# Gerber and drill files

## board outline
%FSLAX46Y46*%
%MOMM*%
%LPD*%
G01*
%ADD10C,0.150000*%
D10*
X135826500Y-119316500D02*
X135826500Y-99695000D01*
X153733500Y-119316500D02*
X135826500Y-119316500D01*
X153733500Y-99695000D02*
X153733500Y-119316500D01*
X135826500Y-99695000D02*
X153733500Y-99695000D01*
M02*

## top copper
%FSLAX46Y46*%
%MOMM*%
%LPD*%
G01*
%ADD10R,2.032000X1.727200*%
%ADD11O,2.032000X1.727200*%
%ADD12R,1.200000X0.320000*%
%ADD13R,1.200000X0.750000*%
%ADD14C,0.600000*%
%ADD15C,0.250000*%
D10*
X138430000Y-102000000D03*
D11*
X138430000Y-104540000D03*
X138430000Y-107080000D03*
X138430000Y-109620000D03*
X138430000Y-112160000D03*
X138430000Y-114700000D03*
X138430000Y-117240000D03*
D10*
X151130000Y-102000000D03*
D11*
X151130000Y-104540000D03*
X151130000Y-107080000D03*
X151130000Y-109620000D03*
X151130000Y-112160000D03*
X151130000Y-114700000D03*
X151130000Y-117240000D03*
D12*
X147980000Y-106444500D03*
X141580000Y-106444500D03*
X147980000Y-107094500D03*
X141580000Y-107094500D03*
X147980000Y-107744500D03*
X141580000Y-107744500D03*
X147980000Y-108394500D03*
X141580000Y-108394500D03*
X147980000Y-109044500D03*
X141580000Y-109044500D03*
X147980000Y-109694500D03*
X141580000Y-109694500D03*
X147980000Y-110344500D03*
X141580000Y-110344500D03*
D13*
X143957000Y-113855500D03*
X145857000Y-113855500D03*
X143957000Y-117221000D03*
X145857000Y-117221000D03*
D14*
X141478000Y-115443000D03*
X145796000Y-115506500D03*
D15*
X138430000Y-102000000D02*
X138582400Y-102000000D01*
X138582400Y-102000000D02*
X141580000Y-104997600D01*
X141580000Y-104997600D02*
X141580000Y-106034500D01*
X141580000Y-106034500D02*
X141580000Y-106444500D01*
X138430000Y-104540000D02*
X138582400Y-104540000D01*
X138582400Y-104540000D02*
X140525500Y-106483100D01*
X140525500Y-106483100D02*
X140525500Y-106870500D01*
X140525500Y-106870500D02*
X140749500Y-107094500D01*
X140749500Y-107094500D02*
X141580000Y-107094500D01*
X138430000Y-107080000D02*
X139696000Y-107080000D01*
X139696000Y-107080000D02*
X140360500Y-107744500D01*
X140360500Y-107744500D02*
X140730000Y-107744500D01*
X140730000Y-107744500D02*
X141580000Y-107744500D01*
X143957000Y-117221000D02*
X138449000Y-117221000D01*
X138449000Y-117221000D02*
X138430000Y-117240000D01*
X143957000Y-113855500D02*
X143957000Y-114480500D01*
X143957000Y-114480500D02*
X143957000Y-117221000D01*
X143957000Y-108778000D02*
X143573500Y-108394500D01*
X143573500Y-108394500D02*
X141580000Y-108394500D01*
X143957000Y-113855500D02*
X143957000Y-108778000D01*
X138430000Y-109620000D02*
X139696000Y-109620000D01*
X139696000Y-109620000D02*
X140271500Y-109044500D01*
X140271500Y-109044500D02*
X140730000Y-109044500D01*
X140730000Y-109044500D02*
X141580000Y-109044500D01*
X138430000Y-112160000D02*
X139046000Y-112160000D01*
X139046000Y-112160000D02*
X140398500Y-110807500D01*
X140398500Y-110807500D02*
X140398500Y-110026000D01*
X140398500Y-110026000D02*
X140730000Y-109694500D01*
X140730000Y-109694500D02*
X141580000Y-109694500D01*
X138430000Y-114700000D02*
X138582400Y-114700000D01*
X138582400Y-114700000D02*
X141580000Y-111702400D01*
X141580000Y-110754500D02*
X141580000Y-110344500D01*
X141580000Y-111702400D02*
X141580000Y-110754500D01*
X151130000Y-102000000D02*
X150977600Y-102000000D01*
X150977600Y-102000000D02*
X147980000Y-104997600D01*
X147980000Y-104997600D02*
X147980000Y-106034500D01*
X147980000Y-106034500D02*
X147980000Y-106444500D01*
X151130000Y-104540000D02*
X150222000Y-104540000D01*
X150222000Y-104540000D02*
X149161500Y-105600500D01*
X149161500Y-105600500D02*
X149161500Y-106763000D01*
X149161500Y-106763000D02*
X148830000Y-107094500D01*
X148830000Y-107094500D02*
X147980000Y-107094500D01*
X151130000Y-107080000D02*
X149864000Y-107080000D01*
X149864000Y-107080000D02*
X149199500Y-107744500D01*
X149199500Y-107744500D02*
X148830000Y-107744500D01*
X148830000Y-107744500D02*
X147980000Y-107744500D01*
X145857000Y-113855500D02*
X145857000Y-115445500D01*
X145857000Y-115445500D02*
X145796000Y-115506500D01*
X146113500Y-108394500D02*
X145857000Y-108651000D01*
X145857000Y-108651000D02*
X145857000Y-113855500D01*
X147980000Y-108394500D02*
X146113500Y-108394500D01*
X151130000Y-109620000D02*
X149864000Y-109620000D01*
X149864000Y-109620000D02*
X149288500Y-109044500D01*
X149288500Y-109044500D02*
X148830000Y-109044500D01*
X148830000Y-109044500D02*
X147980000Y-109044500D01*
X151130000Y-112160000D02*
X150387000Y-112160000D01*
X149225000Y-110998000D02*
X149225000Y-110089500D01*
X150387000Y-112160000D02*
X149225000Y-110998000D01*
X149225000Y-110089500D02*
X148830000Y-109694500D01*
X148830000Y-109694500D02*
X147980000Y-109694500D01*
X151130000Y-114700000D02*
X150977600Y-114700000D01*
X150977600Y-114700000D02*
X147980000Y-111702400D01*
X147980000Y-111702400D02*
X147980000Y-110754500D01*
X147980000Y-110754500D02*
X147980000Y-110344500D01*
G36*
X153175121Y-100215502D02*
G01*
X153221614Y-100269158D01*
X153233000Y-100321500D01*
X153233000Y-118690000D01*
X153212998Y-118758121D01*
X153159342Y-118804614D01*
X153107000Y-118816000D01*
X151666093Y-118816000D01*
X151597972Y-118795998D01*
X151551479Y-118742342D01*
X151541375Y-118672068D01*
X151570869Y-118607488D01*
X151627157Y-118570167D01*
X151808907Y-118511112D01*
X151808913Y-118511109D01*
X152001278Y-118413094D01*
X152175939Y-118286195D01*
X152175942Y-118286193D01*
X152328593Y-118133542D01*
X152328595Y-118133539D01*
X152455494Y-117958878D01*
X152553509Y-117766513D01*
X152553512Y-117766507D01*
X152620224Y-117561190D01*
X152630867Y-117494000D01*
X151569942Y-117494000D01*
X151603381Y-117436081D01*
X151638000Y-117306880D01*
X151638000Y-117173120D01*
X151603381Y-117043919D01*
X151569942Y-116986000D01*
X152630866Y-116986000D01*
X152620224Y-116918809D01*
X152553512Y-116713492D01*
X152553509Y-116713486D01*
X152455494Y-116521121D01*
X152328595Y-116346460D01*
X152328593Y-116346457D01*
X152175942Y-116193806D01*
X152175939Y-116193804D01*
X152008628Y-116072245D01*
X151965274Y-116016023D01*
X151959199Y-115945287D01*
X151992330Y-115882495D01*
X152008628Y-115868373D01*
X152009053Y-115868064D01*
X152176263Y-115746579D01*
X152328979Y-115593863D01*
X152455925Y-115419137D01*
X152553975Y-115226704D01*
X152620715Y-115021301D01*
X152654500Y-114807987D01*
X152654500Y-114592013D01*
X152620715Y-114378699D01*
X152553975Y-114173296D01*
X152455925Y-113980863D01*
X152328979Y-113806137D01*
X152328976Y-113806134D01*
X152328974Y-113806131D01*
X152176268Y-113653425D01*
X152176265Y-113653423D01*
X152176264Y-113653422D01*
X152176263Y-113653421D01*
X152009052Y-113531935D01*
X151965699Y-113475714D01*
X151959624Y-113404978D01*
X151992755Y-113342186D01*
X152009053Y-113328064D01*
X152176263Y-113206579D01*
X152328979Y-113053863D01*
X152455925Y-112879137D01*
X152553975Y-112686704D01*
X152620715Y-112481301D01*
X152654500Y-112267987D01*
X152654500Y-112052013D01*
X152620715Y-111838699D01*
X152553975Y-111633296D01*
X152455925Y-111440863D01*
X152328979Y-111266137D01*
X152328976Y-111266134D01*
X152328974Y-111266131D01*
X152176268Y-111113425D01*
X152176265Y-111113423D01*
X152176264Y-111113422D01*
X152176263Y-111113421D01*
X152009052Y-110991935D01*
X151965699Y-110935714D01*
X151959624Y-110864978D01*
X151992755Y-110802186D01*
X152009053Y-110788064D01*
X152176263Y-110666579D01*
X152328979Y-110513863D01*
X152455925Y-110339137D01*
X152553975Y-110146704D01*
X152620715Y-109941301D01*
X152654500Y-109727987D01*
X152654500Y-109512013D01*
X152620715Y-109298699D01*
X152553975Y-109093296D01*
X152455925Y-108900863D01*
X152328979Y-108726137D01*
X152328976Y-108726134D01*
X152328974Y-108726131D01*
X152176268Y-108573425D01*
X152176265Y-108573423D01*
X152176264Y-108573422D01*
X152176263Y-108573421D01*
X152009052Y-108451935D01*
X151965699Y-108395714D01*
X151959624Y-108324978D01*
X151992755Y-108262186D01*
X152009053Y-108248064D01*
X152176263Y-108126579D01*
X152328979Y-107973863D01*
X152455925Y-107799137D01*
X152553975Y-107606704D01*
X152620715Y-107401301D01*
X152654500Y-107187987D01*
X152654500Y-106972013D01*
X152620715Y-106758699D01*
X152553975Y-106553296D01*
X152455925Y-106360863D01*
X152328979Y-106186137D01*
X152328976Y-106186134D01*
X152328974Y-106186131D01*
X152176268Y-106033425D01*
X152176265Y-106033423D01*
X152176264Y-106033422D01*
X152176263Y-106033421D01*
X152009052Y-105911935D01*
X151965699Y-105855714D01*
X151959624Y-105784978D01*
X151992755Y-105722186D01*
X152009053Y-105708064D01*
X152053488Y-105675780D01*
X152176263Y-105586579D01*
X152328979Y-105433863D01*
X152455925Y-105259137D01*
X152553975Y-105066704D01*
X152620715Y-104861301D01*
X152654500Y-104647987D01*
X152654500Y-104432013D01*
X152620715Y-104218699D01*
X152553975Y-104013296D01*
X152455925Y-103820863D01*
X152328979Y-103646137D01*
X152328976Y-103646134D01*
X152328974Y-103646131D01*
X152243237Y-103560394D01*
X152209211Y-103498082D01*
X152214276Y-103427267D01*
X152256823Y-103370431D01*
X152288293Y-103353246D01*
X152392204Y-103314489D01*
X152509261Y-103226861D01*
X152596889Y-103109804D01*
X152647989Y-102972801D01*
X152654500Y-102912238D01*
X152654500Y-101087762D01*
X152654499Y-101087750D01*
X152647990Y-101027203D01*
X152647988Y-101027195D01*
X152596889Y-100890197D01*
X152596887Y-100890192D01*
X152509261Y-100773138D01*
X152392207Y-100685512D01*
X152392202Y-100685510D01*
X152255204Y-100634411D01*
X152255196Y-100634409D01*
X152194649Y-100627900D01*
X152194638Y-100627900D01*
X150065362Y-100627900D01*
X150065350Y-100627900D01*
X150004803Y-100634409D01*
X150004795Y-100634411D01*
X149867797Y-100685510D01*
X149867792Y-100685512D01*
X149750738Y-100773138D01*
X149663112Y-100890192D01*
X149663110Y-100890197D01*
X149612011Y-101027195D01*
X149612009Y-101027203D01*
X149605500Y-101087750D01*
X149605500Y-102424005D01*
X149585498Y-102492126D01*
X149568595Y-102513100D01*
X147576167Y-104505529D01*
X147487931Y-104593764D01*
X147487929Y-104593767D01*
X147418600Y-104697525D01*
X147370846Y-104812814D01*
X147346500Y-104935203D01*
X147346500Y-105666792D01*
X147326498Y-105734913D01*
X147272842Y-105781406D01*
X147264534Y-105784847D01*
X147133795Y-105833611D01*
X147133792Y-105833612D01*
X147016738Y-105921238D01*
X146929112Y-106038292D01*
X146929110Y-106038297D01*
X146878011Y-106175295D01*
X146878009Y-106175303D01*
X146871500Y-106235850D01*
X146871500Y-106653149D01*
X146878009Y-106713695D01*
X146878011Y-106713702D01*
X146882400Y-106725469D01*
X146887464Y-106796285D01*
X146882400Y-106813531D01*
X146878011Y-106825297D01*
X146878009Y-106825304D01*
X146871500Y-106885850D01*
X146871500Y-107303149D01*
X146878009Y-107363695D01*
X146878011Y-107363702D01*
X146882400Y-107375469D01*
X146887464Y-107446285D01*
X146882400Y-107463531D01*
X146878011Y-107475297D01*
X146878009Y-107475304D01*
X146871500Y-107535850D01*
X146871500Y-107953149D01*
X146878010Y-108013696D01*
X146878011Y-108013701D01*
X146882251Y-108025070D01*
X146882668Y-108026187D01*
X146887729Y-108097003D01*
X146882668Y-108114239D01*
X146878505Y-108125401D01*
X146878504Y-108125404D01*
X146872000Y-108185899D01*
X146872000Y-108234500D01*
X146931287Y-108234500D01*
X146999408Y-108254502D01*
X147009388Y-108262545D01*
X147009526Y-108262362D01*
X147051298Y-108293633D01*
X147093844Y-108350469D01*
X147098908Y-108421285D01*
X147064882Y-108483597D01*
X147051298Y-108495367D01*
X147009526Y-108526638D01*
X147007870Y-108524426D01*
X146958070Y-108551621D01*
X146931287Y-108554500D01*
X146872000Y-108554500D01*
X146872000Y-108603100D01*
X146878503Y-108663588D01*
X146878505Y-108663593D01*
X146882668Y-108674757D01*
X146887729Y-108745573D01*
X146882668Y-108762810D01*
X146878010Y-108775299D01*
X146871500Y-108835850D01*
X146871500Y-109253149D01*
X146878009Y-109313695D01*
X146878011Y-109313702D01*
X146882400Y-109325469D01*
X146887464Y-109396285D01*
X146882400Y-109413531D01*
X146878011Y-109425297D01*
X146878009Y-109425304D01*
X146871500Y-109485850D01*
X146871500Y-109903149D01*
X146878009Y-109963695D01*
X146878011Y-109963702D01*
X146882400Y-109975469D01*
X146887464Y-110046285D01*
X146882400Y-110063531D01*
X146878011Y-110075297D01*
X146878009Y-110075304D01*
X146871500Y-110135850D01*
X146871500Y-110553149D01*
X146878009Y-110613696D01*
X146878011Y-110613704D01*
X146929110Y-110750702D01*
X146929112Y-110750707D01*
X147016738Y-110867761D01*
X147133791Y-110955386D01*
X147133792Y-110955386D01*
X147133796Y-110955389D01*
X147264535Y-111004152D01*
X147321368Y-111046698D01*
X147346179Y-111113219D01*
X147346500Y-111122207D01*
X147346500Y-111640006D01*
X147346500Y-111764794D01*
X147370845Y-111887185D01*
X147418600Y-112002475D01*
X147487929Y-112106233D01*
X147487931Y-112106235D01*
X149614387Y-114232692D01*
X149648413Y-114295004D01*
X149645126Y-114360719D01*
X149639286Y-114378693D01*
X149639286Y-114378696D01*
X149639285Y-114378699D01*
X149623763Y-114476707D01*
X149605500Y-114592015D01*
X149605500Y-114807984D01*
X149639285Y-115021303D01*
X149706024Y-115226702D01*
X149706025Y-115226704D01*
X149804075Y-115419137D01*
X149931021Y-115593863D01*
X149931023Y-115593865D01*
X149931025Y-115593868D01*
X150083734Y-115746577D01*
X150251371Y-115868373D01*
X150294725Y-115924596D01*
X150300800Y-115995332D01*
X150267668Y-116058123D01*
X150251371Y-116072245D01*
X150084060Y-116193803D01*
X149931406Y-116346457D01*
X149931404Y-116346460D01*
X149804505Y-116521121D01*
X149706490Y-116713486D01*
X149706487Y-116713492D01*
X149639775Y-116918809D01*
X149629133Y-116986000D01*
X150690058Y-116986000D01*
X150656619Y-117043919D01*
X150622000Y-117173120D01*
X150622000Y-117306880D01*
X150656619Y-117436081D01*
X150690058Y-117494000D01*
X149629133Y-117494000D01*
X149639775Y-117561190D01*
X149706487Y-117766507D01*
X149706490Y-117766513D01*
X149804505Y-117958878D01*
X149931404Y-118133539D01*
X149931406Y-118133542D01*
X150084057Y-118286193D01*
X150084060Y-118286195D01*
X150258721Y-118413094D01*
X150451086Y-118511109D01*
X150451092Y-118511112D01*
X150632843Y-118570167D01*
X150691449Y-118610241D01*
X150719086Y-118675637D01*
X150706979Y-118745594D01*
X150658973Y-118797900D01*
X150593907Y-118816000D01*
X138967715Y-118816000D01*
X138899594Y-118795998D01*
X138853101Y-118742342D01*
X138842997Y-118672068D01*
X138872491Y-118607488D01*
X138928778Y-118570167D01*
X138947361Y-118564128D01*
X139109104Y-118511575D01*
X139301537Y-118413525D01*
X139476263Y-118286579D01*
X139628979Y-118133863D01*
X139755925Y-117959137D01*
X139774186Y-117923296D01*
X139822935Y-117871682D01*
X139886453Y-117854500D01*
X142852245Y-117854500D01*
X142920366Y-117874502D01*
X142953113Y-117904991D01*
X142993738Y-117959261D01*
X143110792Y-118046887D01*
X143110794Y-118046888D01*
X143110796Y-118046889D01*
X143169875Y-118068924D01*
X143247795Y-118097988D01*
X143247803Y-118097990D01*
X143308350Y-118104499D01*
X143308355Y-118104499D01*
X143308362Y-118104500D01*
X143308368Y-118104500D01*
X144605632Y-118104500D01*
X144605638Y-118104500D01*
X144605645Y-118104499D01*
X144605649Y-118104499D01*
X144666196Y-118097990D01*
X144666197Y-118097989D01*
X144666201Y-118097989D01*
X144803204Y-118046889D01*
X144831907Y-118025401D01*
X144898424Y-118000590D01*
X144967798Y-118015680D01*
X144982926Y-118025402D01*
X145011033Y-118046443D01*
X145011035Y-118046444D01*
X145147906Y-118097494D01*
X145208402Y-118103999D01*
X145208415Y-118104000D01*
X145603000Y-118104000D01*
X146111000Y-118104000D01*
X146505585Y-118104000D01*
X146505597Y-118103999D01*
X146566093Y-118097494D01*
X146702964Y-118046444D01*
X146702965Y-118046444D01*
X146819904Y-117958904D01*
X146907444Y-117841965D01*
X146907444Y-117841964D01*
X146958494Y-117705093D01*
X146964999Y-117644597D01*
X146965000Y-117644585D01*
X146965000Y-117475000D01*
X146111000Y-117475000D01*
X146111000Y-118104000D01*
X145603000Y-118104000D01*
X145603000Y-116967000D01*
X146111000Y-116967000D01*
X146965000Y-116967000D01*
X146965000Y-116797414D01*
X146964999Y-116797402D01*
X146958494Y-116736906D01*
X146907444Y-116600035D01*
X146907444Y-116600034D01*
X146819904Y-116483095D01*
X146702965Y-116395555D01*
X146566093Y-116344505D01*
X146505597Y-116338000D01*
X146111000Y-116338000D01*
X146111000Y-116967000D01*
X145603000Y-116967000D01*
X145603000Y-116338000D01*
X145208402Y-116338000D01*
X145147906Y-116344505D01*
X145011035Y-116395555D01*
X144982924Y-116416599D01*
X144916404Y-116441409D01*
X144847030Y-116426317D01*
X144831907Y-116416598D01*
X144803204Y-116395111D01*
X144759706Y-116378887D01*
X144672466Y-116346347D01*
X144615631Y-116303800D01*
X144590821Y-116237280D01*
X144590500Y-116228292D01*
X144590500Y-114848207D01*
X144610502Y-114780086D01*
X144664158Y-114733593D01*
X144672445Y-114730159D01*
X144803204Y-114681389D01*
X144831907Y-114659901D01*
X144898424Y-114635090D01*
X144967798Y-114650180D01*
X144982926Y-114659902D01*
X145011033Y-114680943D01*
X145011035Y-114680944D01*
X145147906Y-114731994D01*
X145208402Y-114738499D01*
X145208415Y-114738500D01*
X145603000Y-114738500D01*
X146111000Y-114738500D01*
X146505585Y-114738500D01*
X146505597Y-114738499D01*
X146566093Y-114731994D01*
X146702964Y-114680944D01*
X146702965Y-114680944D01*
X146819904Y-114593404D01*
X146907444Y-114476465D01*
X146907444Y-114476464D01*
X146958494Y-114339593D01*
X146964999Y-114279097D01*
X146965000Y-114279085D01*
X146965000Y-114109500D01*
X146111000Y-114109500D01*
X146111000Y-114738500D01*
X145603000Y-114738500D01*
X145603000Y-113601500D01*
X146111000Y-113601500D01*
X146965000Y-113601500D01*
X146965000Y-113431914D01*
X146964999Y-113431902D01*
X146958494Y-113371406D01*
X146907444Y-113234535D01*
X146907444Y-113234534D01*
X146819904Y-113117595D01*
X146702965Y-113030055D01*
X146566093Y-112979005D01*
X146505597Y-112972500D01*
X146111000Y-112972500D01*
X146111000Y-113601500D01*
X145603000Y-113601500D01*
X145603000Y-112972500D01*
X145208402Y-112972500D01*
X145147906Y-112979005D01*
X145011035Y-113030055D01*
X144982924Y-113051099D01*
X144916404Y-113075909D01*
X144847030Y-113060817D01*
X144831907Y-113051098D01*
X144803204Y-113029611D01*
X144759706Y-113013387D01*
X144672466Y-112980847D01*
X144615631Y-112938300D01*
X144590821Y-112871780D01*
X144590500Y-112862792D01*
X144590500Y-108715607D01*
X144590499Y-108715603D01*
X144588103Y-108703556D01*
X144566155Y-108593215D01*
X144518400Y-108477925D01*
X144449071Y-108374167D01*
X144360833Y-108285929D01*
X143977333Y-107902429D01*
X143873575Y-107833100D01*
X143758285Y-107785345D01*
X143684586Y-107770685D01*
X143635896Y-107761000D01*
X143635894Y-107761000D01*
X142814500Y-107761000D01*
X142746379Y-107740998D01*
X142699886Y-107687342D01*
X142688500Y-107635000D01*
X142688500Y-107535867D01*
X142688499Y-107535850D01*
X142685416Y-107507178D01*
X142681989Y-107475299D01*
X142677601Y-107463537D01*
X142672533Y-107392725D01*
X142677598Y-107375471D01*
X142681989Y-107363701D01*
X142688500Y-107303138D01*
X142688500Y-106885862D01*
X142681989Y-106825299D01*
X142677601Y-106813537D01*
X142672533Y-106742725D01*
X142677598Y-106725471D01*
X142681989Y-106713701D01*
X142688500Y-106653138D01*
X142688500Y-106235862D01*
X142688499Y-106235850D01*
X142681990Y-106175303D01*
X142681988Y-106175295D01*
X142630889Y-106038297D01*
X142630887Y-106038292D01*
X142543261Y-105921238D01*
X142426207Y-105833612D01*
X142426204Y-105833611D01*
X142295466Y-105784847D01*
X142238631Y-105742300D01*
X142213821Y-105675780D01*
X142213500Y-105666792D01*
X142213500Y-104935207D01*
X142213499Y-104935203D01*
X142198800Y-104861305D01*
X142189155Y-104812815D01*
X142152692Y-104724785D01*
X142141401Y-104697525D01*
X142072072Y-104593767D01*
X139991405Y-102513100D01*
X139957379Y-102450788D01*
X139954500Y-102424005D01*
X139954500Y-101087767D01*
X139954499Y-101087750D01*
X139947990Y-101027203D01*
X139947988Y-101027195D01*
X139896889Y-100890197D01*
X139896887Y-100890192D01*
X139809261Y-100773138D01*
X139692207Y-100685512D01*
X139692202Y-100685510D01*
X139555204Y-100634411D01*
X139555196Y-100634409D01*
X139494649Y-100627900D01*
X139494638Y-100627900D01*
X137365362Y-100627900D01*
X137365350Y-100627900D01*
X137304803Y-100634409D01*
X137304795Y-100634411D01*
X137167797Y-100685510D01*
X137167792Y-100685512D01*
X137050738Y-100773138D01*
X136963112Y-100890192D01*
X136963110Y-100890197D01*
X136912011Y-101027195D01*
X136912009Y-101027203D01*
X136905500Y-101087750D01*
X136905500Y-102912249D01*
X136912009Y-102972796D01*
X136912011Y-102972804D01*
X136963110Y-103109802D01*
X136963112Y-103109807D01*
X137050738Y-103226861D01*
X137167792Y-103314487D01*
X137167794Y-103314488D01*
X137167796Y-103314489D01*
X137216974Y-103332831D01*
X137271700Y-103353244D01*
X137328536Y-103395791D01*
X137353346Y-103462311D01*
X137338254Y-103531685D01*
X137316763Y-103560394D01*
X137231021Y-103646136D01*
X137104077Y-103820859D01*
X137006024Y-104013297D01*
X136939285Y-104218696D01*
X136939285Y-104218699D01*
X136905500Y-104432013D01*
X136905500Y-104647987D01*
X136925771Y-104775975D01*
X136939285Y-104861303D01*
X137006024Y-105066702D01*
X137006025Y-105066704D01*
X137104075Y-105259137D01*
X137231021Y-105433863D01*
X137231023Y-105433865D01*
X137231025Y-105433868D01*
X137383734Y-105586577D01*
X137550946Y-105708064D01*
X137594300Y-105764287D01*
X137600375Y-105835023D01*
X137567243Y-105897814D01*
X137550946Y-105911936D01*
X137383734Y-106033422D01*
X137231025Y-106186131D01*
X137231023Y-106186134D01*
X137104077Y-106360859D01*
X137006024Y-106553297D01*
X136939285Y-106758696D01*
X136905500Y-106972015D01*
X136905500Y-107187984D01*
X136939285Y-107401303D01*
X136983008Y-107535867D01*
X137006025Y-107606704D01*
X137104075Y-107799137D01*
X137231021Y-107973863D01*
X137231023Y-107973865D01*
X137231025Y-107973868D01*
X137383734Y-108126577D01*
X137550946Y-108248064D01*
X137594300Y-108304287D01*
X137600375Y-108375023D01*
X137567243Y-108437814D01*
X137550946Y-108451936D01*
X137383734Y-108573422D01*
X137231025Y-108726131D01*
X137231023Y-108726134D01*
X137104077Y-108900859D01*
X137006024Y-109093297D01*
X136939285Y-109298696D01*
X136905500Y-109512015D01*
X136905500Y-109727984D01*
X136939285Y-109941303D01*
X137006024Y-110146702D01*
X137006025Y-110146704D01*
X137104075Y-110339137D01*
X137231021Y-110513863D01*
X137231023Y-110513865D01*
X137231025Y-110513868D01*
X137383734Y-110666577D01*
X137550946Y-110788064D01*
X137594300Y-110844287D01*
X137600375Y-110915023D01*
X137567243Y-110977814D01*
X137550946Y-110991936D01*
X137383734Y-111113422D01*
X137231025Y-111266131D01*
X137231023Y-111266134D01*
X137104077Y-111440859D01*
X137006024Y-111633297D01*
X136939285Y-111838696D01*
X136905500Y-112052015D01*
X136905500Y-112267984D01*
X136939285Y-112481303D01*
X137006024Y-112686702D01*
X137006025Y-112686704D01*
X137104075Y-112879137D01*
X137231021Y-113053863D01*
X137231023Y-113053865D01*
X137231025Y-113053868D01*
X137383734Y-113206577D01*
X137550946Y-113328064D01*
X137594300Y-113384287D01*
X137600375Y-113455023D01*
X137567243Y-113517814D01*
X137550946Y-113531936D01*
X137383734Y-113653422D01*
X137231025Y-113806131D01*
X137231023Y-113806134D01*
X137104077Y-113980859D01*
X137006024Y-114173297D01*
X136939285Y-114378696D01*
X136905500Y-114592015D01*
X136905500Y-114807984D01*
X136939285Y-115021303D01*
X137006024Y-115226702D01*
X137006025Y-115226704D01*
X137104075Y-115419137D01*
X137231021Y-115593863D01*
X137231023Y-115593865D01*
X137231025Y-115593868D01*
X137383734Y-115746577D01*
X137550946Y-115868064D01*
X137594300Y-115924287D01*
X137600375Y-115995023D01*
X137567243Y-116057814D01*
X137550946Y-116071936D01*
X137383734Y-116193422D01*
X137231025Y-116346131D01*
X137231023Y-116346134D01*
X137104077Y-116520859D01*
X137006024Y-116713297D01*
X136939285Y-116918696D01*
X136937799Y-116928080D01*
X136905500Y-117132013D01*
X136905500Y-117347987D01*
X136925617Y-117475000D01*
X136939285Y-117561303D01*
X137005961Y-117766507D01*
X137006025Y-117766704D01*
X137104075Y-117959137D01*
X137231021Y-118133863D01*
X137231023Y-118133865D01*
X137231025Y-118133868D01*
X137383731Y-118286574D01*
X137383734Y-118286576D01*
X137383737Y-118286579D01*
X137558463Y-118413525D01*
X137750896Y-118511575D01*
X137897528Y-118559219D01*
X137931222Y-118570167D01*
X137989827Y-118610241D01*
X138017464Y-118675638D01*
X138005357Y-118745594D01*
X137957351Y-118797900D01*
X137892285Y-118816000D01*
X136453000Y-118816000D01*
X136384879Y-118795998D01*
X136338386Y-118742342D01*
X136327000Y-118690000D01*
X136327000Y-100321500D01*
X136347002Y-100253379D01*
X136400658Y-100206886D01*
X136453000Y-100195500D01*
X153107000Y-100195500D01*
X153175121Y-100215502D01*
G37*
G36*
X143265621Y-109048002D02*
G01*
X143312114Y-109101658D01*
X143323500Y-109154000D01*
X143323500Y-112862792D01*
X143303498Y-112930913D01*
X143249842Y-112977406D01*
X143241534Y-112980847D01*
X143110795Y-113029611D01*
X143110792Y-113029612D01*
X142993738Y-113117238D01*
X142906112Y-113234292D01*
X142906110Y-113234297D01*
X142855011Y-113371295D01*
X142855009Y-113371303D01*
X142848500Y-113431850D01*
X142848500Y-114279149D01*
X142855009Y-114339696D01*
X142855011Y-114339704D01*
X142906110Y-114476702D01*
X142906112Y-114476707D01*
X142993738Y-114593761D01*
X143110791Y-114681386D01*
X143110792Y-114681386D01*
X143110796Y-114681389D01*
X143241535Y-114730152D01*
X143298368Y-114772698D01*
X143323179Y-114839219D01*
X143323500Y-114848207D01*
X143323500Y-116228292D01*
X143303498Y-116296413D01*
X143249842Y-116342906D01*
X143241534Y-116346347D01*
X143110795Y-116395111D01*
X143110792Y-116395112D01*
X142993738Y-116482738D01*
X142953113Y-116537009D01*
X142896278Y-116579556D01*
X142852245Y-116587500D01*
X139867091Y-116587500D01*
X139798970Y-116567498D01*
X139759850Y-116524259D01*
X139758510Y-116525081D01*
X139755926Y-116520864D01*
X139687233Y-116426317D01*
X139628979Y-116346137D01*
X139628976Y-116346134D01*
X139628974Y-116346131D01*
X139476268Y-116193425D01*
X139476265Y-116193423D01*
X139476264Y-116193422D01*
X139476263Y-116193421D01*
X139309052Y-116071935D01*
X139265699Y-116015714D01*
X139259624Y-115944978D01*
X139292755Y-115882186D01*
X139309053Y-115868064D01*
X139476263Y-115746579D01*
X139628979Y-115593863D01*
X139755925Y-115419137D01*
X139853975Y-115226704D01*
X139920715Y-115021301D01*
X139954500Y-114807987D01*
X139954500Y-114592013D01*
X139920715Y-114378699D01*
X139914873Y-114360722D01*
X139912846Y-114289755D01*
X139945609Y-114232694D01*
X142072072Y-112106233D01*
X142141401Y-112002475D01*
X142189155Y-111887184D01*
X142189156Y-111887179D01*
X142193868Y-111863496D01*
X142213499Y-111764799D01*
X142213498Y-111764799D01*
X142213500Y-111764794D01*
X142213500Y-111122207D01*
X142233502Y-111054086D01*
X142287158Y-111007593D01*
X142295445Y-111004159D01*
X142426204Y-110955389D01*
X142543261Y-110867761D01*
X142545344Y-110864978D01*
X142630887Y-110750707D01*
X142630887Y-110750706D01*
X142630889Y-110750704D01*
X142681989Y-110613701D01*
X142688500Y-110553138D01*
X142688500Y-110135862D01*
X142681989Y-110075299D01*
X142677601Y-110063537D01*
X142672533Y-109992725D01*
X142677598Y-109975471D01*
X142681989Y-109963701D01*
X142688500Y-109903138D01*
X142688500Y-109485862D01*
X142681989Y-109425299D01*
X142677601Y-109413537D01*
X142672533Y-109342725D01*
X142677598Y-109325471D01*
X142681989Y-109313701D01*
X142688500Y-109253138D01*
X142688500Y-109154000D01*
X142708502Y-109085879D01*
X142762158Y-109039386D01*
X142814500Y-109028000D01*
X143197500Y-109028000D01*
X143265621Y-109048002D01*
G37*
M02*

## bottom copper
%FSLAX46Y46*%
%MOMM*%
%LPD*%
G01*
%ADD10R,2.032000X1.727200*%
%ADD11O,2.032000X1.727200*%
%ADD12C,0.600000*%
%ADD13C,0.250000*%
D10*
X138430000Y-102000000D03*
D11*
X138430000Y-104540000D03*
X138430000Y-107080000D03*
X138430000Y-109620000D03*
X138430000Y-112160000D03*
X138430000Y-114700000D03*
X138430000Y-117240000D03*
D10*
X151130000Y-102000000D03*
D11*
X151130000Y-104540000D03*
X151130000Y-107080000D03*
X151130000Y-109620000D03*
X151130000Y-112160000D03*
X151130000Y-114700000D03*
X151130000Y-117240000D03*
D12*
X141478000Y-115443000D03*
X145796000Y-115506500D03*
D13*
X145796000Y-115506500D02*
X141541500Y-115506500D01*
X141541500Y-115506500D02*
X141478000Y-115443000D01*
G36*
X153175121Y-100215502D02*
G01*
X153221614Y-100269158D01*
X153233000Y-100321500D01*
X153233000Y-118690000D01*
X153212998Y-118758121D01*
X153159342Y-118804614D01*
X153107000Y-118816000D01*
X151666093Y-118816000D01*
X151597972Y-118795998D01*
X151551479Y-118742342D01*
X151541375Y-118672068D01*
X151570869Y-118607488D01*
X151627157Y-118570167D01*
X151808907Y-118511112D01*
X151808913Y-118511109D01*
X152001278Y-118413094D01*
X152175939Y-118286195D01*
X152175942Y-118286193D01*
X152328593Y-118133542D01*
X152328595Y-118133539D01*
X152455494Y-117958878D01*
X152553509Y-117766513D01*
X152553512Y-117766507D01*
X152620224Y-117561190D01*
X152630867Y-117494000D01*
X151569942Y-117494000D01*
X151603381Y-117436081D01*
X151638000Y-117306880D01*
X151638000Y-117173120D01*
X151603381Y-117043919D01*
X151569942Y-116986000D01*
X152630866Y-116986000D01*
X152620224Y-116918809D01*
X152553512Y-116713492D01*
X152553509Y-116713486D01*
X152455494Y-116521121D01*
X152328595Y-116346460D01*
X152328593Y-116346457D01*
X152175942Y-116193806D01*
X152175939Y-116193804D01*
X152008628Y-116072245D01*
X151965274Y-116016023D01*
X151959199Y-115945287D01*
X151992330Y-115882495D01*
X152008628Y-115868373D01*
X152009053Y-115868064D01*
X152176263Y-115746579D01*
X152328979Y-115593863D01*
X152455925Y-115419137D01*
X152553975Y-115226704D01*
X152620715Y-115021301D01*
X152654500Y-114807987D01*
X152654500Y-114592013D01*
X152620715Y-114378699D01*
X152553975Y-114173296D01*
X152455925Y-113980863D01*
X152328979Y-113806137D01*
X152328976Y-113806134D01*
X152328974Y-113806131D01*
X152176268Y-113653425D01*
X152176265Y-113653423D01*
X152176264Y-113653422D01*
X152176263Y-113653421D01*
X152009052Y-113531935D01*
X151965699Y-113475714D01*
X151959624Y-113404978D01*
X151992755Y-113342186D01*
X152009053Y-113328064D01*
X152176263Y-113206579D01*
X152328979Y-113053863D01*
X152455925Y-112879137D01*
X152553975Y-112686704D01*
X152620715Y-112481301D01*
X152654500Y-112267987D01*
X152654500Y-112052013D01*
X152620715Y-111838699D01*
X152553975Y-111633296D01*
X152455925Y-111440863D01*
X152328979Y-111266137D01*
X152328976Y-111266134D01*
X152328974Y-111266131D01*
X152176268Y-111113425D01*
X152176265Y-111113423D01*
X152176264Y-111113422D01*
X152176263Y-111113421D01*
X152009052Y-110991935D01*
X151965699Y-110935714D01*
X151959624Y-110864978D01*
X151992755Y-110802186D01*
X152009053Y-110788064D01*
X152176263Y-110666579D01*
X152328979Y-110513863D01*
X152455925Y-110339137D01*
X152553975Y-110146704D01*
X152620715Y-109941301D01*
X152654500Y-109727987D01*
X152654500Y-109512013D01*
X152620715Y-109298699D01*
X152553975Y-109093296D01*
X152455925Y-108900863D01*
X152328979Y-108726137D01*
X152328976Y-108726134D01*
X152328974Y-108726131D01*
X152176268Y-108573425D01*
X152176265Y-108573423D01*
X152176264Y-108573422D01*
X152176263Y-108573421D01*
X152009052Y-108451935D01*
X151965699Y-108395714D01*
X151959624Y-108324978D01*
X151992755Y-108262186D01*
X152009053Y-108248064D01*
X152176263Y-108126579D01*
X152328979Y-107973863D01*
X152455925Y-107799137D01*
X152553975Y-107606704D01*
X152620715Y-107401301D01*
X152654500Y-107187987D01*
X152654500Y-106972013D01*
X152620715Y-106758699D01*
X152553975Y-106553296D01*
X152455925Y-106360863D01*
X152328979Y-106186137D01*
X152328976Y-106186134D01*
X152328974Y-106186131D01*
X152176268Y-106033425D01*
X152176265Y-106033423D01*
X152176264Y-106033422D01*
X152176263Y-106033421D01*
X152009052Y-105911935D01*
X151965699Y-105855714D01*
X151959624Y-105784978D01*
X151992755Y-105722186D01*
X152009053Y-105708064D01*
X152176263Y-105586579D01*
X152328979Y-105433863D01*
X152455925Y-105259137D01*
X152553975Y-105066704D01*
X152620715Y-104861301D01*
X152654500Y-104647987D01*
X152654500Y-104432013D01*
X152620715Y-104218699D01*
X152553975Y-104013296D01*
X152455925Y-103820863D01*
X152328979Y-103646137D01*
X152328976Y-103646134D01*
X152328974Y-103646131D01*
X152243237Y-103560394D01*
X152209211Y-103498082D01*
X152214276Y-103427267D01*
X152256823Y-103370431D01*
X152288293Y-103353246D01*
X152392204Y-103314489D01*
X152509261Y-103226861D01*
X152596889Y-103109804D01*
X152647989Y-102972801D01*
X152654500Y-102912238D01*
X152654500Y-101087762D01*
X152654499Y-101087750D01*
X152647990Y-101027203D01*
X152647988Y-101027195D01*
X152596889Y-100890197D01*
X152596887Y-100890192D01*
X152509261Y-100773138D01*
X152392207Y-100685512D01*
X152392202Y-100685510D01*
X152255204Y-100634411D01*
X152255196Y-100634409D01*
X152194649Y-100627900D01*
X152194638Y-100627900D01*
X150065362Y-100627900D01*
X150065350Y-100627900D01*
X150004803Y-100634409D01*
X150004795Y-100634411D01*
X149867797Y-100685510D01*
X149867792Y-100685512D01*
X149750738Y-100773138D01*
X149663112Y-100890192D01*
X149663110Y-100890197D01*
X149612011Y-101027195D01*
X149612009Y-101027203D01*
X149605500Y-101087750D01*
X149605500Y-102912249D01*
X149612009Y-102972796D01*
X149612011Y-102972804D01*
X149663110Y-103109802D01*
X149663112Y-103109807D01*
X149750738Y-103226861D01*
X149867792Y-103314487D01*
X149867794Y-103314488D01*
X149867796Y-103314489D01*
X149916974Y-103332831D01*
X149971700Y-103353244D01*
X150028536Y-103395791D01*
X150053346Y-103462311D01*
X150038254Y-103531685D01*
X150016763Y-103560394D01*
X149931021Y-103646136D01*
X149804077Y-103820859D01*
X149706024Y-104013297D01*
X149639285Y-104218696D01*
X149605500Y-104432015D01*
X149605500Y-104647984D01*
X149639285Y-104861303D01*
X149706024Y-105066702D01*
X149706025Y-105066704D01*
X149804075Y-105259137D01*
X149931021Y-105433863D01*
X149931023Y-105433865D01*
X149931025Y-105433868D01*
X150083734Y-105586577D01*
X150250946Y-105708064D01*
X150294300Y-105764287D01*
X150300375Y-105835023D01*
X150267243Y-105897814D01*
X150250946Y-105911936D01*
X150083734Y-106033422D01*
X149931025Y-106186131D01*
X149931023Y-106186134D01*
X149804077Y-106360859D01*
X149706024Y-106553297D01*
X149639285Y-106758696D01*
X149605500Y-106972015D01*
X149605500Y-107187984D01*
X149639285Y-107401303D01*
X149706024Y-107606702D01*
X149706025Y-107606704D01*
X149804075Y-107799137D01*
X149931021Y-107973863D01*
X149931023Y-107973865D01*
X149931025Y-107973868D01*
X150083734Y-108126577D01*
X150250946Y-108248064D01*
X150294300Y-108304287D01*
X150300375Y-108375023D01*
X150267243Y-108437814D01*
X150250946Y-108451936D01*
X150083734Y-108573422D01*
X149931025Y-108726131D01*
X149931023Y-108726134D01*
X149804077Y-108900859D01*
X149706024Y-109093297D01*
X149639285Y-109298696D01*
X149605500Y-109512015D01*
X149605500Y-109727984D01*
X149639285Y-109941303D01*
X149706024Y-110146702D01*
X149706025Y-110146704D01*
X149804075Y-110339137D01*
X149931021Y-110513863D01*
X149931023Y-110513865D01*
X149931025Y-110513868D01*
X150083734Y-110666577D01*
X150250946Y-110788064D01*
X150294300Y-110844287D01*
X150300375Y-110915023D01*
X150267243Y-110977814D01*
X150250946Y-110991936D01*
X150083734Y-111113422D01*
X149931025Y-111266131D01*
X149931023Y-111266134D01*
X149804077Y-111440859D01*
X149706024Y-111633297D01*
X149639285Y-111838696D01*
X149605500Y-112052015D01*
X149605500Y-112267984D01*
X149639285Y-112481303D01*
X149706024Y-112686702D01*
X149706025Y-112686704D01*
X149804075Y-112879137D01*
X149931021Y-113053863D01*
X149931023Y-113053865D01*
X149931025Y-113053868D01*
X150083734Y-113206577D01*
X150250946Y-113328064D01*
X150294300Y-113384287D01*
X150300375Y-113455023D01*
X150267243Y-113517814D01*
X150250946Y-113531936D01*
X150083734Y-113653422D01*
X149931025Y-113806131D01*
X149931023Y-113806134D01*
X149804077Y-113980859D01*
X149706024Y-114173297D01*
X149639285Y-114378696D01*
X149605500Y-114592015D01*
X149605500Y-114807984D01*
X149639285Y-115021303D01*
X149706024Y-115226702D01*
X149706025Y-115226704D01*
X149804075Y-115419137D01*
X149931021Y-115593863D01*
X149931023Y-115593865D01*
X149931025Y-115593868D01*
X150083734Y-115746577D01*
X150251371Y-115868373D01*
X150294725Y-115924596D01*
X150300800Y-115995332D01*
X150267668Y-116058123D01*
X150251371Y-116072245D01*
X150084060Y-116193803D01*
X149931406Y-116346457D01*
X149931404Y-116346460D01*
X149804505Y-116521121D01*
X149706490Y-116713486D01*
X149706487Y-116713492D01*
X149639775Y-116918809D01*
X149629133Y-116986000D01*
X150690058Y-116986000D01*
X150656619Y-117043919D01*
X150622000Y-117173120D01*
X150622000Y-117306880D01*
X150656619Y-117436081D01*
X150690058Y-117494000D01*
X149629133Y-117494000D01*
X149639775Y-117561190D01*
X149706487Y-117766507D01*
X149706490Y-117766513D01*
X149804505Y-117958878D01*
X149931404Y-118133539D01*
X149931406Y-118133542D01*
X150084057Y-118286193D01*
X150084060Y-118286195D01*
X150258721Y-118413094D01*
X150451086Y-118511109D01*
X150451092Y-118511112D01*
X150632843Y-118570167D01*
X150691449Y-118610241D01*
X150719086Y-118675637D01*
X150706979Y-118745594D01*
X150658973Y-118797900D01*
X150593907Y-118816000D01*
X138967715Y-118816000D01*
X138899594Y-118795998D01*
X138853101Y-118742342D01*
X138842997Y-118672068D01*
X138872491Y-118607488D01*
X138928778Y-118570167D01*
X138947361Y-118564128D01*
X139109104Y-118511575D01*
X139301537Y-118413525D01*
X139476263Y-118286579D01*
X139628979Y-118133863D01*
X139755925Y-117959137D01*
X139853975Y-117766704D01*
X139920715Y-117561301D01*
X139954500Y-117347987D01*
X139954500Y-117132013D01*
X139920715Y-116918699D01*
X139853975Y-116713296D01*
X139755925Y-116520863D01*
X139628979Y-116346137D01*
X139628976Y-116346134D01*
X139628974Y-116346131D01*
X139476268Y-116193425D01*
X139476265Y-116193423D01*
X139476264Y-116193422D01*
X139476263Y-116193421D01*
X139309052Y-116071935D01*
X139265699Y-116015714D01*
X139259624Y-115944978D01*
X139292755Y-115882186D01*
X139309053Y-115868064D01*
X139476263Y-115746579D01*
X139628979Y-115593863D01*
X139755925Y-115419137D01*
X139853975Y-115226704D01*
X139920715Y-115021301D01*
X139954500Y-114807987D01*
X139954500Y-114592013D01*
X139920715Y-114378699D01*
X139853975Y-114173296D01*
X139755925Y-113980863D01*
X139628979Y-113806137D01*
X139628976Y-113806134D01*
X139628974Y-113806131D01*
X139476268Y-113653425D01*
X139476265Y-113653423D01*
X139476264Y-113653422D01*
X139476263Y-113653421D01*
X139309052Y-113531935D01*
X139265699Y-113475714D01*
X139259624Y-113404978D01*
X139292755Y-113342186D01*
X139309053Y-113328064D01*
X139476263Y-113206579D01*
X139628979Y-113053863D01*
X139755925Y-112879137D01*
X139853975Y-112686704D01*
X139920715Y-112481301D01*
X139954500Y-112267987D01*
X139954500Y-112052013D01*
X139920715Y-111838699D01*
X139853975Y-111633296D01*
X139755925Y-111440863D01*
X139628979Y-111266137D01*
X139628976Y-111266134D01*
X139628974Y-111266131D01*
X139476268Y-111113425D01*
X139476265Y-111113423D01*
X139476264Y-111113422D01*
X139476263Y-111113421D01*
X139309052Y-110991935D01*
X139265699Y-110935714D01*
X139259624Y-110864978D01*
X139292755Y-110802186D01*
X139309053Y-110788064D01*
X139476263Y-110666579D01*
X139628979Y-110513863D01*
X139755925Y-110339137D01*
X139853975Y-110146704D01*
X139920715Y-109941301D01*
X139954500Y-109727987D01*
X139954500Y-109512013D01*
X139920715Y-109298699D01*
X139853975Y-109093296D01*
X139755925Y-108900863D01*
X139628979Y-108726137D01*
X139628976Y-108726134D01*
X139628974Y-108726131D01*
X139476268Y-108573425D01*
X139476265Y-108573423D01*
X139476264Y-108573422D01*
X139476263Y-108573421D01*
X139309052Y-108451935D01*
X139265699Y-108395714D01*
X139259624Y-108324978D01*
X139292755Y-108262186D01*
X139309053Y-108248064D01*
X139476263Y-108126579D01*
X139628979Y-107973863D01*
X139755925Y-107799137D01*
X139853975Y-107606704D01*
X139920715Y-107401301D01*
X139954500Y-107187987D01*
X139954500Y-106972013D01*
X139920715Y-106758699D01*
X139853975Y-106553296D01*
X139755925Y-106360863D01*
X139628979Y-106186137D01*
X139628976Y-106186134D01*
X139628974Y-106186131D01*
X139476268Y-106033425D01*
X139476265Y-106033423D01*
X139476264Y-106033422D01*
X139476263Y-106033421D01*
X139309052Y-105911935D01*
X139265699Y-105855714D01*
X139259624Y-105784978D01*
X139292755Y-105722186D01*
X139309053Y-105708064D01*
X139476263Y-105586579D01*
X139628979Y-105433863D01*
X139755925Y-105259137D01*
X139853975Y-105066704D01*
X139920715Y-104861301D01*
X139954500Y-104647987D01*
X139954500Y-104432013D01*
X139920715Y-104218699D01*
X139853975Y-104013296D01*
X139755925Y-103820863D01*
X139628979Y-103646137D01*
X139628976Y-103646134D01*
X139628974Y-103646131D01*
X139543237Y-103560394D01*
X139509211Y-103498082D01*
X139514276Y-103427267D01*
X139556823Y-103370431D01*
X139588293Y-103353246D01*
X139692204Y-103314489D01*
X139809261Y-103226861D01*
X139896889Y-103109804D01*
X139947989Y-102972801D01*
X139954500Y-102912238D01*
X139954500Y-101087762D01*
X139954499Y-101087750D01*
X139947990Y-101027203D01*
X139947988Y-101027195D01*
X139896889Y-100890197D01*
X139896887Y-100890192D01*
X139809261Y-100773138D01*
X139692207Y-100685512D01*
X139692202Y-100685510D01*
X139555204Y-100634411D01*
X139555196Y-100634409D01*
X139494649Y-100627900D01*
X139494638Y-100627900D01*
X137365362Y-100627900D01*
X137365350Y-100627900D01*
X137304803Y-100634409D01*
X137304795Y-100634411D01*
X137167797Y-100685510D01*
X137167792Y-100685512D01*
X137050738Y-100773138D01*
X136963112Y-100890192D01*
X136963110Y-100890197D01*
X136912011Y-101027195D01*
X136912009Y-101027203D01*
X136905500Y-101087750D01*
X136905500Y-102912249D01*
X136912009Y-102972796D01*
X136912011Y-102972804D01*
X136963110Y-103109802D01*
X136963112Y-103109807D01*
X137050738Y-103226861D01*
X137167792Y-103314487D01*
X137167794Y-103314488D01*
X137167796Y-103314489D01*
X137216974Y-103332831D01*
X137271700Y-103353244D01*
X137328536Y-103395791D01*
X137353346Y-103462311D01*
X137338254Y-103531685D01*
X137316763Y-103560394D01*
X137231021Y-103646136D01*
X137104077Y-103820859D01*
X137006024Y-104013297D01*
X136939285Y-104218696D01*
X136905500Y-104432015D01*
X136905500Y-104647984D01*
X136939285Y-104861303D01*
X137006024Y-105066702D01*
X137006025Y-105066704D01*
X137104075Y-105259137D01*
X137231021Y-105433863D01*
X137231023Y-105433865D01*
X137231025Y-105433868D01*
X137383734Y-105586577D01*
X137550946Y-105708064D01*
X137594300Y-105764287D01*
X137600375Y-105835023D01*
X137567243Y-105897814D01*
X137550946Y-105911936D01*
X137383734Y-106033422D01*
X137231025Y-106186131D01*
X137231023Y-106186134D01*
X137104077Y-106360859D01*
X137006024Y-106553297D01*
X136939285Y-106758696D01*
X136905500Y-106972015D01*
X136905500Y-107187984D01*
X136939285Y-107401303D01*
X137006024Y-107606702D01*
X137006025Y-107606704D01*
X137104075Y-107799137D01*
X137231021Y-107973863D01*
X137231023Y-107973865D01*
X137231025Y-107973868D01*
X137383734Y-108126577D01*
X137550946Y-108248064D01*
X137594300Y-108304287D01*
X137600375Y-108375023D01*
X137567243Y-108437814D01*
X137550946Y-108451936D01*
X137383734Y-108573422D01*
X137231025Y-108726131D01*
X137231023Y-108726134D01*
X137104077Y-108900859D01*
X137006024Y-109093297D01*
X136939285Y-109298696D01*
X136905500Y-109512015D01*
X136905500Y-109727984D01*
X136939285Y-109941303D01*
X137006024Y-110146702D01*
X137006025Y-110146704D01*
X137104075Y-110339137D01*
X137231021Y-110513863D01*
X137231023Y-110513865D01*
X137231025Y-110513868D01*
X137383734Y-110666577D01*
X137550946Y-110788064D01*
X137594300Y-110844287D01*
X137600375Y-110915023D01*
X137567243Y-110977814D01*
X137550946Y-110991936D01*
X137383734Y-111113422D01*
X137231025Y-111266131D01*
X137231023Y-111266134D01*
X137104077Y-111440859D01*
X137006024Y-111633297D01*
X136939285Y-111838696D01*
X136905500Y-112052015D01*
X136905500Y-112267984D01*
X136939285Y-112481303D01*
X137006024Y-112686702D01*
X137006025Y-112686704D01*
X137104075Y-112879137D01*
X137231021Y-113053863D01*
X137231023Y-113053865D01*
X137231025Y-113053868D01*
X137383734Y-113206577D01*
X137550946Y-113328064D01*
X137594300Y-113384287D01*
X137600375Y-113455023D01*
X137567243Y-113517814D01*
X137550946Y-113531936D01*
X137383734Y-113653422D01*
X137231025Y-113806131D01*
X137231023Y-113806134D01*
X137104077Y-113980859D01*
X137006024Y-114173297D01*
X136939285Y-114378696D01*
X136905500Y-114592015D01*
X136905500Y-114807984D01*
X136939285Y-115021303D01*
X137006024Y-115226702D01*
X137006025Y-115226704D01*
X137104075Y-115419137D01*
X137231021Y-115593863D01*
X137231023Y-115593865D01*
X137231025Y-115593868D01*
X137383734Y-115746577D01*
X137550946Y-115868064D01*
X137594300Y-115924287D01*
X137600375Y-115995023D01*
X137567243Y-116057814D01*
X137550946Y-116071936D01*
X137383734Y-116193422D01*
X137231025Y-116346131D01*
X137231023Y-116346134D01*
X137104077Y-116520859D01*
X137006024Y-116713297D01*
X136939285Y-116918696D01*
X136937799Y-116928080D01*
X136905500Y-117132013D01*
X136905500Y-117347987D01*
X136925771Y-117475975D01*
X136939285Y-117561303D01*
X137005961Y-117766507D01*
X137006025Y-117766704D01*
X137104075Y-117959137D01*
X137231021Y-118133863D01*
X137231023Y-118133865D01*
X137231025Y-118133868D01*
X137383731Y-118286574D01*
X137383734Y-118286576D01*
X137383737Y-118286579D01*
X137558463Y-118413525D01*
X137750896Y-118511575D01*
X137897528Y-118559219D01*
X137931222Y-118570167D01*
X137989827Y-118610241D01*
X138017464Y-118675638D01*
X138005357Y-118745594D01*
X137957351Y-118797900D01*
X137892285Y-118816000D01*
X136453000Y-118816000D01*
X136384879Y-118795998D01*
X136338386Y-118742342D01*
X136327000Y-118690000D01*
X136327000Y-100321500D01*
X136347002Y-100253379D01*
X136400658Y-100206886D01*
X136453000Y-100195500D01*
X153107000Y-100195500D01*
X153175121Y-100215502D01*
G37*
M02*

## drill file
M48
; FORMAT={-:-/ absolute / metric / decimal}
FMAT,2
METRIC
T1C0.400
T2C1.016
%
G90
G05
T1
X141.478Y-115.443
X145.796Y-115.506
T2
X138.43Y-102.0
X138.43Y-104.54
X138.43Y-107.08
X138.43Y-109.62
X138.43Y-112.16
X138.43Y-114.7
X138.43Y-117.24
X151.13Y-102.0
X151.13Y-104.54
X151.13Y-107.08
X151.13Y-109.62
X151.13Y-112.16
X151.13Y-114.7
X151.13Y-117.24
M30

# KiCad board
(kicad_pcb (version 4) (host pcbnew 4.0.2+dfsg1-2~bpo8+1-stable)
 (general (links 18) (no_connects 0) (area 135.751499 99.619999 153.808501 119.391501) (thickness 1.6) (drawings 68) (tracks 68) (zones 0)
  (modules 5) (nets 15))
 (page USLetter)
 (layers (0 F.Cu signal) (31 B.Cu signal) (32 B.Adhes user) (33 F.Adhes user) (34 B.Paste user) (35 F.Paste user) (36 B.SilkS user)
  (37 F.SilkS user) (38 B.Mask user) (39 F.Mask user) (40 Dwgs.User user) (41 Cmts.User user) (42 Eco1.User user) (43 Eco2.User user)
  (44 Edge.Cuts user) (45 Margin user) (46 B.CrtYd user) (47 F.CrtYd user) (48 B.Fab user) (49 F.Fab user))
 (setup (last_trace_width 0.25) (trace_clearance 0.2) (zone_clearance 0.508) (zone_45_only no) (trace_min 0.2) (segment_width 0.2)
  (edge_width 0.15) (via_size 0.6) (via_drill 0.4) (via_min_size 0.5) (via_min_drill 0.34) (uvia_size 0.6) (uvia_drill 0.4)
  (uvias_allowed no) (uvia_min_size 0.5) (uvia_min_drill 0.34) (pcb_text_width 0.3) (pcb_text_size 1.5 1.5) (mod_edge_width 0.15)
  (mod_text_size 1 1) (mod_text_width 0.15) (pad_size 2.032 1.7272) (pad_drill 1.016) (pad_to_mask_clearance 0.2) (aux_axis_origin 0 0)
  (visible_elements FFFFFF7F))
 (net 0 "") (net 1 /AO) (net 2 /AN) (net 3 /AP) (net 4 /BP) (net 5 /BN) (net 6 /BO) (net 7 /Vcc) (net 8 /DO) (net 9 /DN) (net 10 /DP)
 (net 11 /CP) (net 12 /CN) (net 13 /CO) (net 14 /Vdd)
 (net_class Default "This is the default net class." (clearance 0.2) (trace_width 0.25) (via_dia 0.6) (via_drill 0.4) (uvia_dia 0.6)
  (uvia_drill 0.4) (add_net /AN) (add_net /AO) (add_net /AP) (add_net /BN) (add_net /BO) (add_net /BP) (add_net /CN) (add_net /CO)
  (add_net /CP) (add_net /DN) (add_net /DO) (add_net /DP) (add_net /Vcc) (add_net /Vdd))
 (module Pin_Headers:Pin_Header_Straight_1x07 (layer F.Cu) (at 138.43 102)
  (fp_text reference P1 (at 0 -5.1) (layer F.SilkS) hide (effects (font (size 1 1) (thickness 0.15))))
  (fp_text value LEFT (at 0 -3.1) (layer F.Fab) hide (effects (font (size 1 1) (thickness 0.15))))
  (pad 1 thru_hole rect (at 0 0) (size 2.032 1.7272) (drill 1.016) (layers *.Cu *.Mask F.SilkS) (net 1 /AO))
  (pad 2 thru_hole oval (at 0 2.54) (size 2.032 1.7272) (drill 1.016) (layers *.Cu *.Mask F.SilkS) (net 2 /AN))
  (pad 3 thru_hole oval (at 0 5.08) (size 2.032 1.7272) (drill 1.016) (layers *.Cu *.Mask F.SilkS) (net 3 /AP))
  (pad 4 thru_hole oval (at 0 7.62) (size 2.032 1.7272) (drill 1.016) (layers *.Cu *.Mask F.SilkS) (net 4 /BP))
  (pad 5 thru_hole oval (at 0 10.16) (size 2.032 1.7272) (drill 1.016) (layers *.Cu *.Mask F.SilkS) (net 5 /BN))
  (pad 6 thru_hole oval (at 0 12.7) (size 2.032 1.7272) (drill 1.016) (layers *.Cu *.Mask F.SilkS) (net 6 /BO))
  (pad 7 thru_hole oval (at 0 15.24) (size 2.032 1.7272) (drill 1.016) (layers *.Cu *.Mask F.SilkS) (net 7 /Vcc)))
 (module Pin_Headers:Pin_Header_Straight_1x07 (layer F.Cu) (at 151.13 102)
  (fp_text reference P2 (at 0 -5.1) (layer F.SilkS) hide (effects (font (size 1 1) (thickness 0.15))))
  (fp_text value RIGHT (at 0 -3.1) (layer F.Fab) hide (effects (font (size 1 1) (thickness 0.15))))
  (pad 1 thru_hole rect (at 0 0) (size 2.032 1.7272) (drill 1.016) (layers *.Cu *.Mask F.SilkS) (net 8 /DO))
  (pad 2 thru_hole oval (at 0 2.54) (size 2.032 1.7272) (drill 1.016) (layers *.Cu *.Mask F.SilkS) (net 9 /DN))
  (pad 3 thru_hole oval (at 0 5.08) (size 2.032 1.7272) (drill 1.016) (layers *.Cu *.Mask F.SilkS) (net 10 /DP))
  (pad 4 thru_hole oval (at 0 7.62) (size 2.032 1.7272) (drill 1.016) (layers *.Cu *.Mask F.SilkS) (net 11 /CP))
  (pad 5 thru_hole oval (at 0 10.16) (size 2.032 1.7272) (drill 1.016) (layers *.Cu *.Mask F.SilkS) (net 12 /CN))
  (pad 6 thru_hole oval (at 0 12.7) (size 2.032 1.7272) (drill 1.016) (layers *.Cu *.Mask F.SilkS) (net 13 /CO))
  (pad 7 thru_hole oval (at 0 15.24) (size 2.032 1.7272) (drill 1.016) (layers *.Cu *.Mask F.SilkS) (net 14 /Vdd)))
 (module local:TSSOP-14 (layer F.Cu) (at 144.78 108.3945 270) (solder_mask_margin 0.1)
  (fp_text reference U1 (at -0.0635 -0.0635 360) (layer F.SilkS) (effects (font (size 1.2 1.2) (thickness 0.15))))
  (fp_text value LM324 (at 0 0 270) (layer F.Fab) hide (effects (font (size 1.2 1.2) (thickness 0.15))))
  (pad 14 smd rect (at -1.95 -3.2 270) (size 0.32 1.2) (layers F.Cu F.Paste F.Mask) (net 8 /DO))
  (pad 1 smd rect (at -1.95 3.2 270) (size 0.32 1.2) (layers F.Cu F.Paste F.Mask) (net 1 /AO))
  (pad 13 smd rect (at -1.3 -3.2 270) (size 0.32 1.2) (layers F.Cu F.Paste F.Mask) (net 9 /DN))
  (pad 2 smd rect (at -1.3 3.2 270) (size 0.32 1.2) (layers F.Cu F.Paste F.Mask) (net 2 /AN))
  (pad 12 smd rect (at -0.65 -3.2 270) (size 0.32 1.2) (layers F.Cu F.Paste F.Mask) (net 10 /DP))
  (pad 3 smd rect (at -0.65 3.2 270) (size 0.32 1.2) (layers F.Cu F.Paste F.Mask) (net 3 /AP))
  (pad 11 smd rect (at 0 -3.2 270) (size 0.32 1.2) (layers F.Cu F.Paste F.Mask) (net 14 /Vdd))
  (pad 4 smd rect (at 0 3.2 270) (size 0.32 1.2) (layers F.Cu F.Paste F.Mask) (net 7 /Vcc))
  (pad 10 smd rect (at 0.65 -3.2 270) (size 0.32 1.2) (layers F.Cu F.Paste F.Mask) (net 11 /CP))
  (pad 5 smd rect (at 0.65 3.2 270) (size 0.32 1.2) (layers F.Cu F.Paste F.Mask) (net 4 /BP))
  (pad 9 smd rect (at 1.3 -3.2 270) (size 0.32 1.2) (layers F.Cu F.Paste F.Mask) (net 12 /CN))
  (pad 6 smd rect (at 1.3 3.2 270) (size 0.32 1.2) (layers F.Cu F.Paste F.Mask) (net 5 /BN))
  (pad 8 smd rect (at 1.95 -3.2 270) (size 0.32 1.2) (layers F.Cu F.Paste F.Mask) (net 13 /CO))
  (pad 7 smd rect (at 1.95 3.2 270) (size 0.32 1.2) (layers F.Cu F.Paste F.Mask) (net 6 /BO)))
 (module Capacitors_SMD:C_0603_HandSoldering (layer F.Cu) (at 144.907 113.8555)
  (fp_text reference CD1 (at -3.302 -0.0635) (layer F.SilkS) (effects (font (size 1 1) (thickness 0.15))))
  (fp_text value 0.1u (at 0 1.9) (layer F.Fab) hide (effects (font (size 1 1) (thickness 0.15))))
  (pad 1 smd rect (at -0.95 0) (size 1.2 0.75) (layers F.Cu F.Paste F.Mask) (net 7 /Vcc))
  (pad 2 smd rect (at 0.95 0) (size 1.2 0.75) (layers F.Cu F.Paste F.Mask) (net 14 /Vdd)))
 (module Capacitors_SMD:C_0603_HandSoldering (layer F.Cu) (at 144.907 117.221)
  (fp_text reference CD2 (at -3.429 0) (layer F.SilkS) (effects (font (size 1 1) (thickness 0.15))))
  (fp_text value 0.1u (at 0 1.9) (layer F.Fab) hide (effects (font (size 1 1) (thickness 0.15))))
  (pad 1 smd rect (at -0.95 0) (size 1.2 0.75) (layers F.Cu F.Paste F.Mask) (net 7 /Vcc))
  (pad 2 smd rect (at 0.95 0) (size 1.2 0.75) (layers F.Cu F.Paste F.Mask) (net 14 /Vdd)))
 (gr_line (start 135.8265 119.3165) (end 135.8265 99.695) (layer Edge.Cuts) (width 0.15))
 (gr_line (start 153.7335 119.3165) (end 135.8265 119.3165) (layer Edge.Cuts) (width 0.15))
 (gr_line (start 153.7335 99.695) (end 153.7335 119.3165) (layer Edge.Cuts) (width 0.15))
 (gr_line (start 135.8265 99.695) (end 153.7335 99.695) (layer Edge.Cuts) (width 0.15))
 (segment (start 138.43 102) (end 138.5824 102) (width 0.25) (layer F.Cu) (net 1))
 (segment (start 138.5824 102) (end 141.58 104.9976) (width 0.25) (layer F.Cu) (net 1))
 (segment (start 141.58 104.9976) (end 141.58 106.0345) (width 0.25) (layer F.Cu) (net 1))
 (segment (start 141.58 106.0345) (end 141.58 106.4445) (width 0.25) (layer F.Cu) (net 1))
 (segment (start 138.43 104.54) (end 138.5824 104.54) (width 0.25) (layer F.Cu) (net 2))
 (segment (start 138.5824 104.54) (end 140.5255 106.4831) (width 0.25) (layer F.Cu) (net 2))
 (segment (start 140.5255 106.4831) (end 140.5255 106.8705) (width 0.25) (layer F.Cu) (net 2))
 (segment (start 140.5255 106.8705) (end 140.7495 107.0945) (width 0.25) (layer F.Cu) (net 2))
 (segment (start 140.7495 107.0945) (end 141.58 107.0945) (width 0.25) (layer F.Cu) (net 2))
 (segment (start 138.43 107.08) (end 139.696 107.08) (width 0.25) (layer F.Cu) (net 3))
 (segment (start 139.696 107.08) (end 140.3605 107.7445) (width 0.25) (layer F.Cu) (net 3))
 (segment (start 140.3605 107.7445) (end 140.73 107.7445) (width 0.25) (layer F.Cu) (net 3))
 (segment (start 140.73 107.7445) (end 141.58 107.7445) (width 0.25) (layer F.Cu) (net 3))
 (segment (start 143.957 117.221) (end 138.449 117.221) (width 0.25) (layer F.Cu) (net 7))
 (segment (start 138.449 117.221) (end 138.43 117.24) (width 0.25) (layer F.Cu) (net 7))
 (segment (start 143.957 113.8555) (end 143.957 114.4805) (width 0.25) (layer F.Cu) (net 7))
 (segment (start 143.957 114.4805) (end 143.957 117.221) (width 0.25) (layer F.Cu) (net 7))
 (segment (start 143.957 108.778) (end 143.5735 108.3945) (width 0.25) (layer F.Cu) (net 7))
 (segment (start 143.5735 108.3945) (end 141.58 108.3945) (width 0.25) (layer F.Cu) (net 7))
 (segment (start 143.957 113.8555) (end 143.957 108.778) (width 0.25) (layer F.Cu) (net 7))
 (segment (start 138.43 109.62) (end 139.696 109.62) (width 0.25) (layer F.Cu) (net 4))
 (segment (start 139.696 109.62) (end 140.2715 109.0445) (width 0.25) (layer F.Cu) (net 4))
 (segment (start 140.2715 109.0445) (end 140.73 109.0445) (width 0.25) (layer F.Cu) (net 4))
 (segment (start 140.73 109.0445) (end 141.58 109.0445) (width 0.25) (layer F.Cu) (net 4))
 (segment (start 138.43 112.16) (end 139.046 112.16) (width 0.25) (layer F.Cu) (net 5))
 (segment (start 139.046 112.16) (end 140.3985 110.8075) (width 0.25) (layer F.Cu) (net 5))
 (segment (start 140.3985 110.8075) (end 140.3985 110.026) (width 0.25) (layer F.Cu) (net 5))
 (segment (start 140.3985 110.026) (end 140.73 109.6945) (width 0.25) (layer F.Cu) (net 5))
 (segment (start 140.73 109.6945) (end 141.58 109.6945) (width 0.25) (layer F.Cu) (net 5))
 (segment (start 138.43 114.7) (end 138.5824 114.7) (width 0.25) (layer F.Cu) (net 6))
 (segment (start 138.5824 114.7) (end 141.58 111.7024) (width 0.25) (layer F.Cu) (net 6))
 (segment (start 141.58 110.7545) (end 141.58 110.3445) (width 0.25) (layer F.Cu) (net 6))
 (segment (start 141.58 111.7024) (end 141.58 110.7545) (width 0.25) (layer F.Cu) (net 6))
 (segment (start 151.13 102) (end 150.9776 102) (width 0.25) (layer F.Cu) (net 8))
 (segment (start 150.9776 102) (end 147.98 104.9976) (width 0.25) (layer F.Cu) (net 8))
 (segment (start 147.98 104.9976) (end 147.98 106.0345) (width 0.25) (layer F.Cu) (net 8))
 (segment (start 147.98 106.0345) (end 147.98 106.4445) (width 0.25) (layer F.Cu) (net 8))
 (segment (start 151.13 104.54) (end 150.222 104.54) (width 0.25) (layer F.Cu) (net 9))
 (segment (start 150.222 104.54) (end 149.1615 105.6005) (width 0.25) (layer F.Cu) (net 9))
 (segment (start 149.1615 105.6005) (end 149.1615 106.763) (width 0.25) (layer F.Cu) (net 9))
 (segment (start 149.1615 106.763) (end 148.83 107.0945) (width 0.25) (layer F.Cu) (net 9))
 (segment (start 148.83 107.0945) (end 147.98 107.0945) (width 0.25) (layer F.Cu) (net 9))
 (segment (start 151.13 107.08) (end 149.864 107.08) (width 0.25) (layer F.Cu) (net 10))
 (segment (start 149.864 107.08) (end 149.1995 107.7445) (width 0.25) (layer F.Cu) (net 10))
 (segment (start 149.1995 107.7445) (end 148.83 107.7445) (width 0.25) (layer F.Cu) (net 10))
 (segment (start 148.83 107.7445) (end 147.98 107.7445) (width 0.25) (layer F.Cu) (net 10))
 (segment (start 145.796 115.5065) (end 141.5415 115.5065) (width 0.25) (layer B.Cu) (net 14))
 (segment (start 141.5415 115.5065) (end 141.478 115.443) (width 0.25) (layer B.Cu) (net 14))
 (via (at 141.478 115.443) (size 0.6) (drill 0.4) (layers F.Cu B.Cu) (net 14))
 (segment (start 145.857 113.8555) (end 145.857 115.4455) (width 0.25) (layer F.Cu) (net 14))
 (segment (start 145.857 115.4455) (end 145.796 115.5065) (width 0.25) (layer F.Cu) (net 14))
 (via (at 145.796 115.5065) (size 0.6) (drill 0.4) (layers F.Cu B.Cu) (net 14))
 (segment (start 146.1135 108.3945) (end 145.857 108.651) (width 0.25) (layer F.Cu) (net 14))
 (segment (start 145.857 108.651) (end 145.857 113.8555) (width 0.25) (layer F.Cu) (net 14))
 (segment (start 147.98 108.3945) (end 146.1135 108.3945) (width 0.25) (layer F.Cu) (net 14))
 (segment (start 151.13 109.62) (end 149.864 109.62) (width 0.25) (layer F.Cu) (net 11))
 (segment (start 149.864 109.62) (end 149.2885 109.0445) (width 0.25) (layer F.Cu) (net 11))
 (segment (start 149.2885 109.0445) (end 148.83 109.0445) (width 0.25) (layer F.Cu) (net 11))
 (segment (start 148.83 109.0445) (end 147.98 109.0445) (width 0.25) (layer F.Cu) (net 11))
 (segment (start 151.13 112.16) (end 150.387 112.16) (width 0.25) (layer F.Cu) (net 12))
 (segment (start 149.225 110.998) (end 149.225 110.0895) (width 0.25) (layer F.Cu) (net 12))
 (segment (start 150.387 112.16) (end 149.225 110.998) (width 0.25) (layer F.Cu) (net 12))
 (segment (start 149.225 110.0895) (end 148.83 109.6945) (width 0.25) (layer F.Cu) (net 12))
 (segment (start 148.83 109.6945) (end 147.98 109.6945) (width 0.25) (layer F.Cu) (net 12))
 (segment (start 151.13 114.7) (end 150.9776 114.7) (width 0.25) (layer F.Cu) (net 13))
 (segment (start 150.9776 114.7) (end 147.98 111.7024) (width 0.25) (layer F.Cu) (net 13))
 (segment (start 147.98 111.7024) (end 147.98 110.7545) (width 0.25) (layer F.Cu) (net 13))
 (segment (start 147.98 110.7545) (end 147.98 110.3445) (width 0.25) (layer F.Cu) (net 13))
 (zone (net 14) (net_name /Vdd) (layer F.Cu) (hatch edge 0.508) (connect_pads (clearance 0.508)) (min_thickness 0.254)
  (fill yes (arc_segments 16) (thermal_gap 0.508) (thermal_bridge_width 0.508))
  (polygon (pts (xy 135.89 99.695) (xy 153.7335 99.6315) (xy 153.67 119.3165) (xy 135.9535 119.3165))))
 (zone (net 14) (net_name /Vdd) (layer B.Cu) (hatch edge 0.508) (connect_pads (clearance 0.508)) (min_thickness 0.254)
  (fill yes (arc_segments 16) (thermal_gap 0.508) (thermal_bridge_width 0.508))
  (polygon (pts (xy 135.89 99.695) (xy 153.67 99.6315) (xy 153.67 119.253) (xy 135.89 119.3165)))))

